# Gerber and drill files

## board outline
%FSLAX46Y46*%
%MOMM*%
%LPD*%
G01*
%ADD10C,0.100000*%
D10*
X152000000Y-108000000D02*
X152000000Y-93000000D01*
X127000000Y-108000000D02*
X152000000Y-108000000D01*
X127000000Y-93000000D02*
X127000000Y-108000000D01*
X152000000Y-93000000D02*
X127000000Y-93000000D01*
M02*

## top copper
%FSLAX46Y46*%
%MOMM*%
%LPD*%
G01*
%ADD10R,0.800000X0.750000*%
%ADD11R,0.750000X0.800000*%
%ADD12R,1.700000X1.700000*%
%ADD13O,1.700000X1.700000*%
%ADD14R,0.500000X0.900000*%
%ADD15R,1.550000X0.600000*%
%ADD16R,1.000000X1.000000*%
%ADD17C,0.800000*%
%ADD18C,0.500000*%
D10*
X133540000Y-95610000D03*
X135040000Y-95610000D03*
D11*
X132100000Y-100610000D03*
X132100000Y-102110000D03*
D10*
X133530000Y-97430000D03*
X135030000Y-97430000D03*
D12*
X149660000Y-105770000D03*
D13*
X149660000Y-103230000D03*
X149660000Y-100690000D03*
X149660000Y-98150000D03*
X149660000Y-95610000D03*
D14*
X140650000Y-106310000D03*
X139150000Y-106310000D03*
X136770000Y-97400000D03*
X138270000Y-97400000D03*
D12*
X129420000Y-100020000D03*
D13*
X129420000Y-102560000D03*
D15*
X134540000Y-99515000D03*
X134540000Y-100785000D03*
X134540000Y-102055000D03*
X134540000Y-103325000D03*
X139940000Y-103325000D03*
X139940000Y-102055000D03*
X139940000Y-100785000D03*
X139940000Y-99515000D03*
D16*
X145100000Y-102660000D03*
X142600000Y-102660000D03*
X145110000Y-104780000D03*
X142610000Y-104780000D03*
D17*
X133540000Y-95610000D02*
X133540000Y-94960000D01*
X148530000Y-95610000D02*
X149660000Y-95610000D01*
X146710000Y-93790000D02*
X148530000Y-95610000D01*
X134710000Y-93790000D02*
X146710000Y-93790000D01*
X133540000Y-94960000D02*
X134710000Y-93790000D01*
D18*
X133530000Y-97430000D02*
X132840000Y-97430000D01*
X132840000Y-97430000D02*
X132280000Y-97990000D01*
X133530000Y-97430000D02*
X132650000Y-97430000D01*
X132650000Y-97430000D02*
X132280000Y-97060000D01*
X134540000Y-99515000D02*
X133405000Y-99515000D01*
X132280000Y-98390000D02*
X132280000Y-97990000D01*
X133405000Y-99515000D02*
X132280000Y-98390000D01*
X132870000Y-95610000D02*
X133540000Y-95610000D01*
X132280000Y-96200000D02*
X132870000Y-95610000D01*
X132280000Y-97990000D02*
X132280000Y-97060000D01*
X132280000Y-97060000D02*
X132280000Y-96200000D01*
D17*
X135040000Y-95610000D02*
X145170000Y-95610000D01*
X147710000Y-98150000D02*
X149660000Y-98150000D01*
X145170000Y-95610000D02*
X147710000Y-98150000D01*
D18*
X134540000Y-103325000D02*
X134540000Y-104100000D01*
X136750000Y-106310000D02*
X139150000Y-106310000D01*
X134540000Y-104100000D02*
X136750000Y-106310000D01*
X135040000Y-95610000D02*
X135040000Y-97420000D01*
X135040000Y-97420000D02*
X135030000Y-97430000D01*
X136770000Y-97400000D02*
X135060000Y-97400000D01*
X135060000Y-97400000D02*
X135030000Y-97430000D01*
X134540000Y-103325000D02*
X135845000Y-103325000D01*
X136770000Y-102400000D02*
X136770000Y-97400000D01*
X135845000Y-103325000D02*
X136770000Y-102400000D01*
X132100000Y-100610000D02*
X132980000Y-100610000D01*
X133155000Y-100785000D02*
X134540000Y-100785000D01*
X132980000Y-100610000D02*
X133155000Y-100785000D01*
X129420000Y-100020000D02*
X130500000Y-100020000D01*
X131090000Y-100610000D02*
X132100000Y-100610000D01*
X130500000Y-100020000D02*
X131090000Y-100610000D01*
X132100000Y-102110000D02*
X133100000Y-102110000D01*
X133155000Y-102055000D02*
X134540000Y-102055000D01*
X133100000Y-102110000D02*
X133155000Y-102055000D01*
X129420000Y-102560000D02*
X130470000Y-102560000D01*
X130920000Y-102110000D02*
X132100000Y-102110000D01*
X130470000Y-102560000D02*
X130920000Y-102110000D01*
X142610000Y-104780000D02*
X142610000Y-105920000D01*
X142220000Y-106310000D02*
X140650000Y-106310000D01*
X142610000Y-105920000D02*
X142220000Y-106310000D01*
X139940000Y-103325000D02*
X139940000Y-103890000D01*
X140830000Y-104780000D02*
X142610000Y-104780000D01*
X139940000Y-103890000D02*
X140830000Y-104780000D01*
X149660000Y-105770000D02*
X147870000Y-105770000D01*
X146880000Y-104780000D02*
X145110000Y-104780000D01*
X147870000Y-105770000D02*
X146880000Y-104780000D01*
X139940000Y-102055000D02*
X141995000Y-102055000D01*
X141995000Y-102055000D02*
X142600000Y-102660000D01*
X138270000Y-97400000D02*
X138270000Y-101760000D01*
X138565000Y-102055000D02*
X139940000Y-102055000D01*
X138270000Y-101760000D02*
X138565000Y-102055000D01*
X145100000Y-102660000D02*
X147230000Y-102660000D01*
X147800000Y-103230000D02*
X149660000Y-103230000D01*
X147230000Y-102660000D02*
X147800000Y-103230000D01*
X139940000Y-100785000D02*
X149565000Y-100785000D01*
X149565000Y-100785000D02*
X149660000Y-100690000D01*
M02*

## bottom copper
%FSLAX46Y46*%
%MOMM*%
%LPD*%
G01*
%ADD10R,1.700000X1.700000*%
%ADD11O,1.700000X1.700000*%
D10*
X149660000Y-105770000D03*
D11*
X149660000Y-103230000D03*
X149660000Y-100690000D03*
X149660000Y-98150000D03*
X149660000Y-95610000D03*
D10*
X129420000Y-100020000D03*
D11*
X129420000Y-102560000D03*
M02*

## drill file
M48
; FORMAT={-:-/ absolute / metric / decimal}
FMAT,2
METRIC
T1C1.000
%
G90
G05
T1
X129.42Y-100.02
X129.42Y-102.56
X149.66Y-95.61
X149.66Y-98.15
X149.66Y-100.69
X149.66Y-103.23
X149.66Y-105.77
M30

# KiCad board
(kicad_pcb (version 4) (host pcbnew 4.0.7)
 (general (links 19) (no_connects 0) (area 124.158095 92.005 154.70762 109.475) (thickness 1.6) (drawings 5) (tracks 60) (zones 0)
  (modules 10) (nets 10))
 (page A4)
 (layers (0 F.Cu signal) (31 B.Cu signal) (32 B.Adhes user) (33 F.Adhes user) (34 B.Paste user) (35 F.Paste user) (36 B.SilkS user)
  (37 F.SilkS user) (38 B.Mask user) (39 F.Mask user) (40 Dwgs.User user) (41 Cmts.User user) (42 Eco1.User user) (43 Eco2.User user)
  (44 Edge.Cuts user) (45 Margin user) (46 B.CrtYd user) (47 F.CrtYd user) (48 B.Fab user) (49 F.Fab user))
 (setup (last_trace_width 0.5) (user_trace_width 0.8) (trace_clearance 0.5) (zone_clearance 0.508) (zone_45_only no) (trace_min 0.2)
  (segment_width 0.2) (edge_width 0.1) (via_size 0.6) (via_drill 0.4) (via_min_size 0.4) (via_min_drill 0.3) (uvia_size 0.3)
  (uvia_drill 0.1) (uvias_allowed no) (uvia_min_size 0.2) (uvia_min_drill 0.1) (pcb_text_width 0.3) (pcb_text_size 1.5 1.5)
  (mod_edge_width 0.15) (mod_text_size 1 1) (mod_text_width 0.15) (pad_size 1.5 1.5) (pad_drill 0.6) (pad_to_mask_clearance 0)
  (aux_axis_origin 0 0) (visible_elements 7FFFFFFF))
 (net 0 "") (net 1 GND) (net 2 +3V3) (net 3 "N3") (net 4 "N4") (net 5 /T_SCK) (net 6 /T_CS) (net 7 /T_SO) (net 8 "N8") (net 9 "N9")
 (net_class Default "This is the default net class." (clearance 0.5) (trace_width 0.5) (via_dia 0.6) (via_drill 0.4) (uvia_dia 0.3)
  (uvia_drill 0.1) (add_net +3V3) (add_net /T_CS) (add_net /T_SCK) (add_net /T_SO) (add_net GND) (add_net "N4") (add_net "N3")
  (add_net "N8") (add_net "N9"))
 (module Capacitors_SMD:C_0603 (layer F.Cu) (at 134.29 95.61 180)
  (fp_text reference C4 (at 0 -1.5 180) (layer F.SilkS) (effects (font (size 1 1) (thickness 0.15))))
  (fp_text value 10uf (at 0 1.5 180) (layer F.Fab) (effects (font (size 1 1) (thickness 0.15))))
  (pad 2 smd rect (at 0.75 0 180) (size 0.8 0.75) (layers F.Cu F.Paste F.Mask) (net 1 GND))
  (pad 1 smd rect (at -0.75 0 180) (size 0.8 0.75) (layers F.Cu F.Paste F.Mask) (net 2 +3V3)))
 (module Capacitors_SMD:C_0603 (layer F.Cu) (at 132.1 101.36 90)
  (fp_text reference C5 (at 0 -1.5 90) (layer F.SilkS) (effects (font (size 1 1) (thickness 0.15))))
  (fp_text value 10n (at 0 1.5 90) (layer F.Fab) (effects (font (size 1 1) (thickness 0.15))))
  (pad 2 smd rect (at 0.75 0 90) (size 0.8 0.75) (layers F.Cu F.Paste F.Mask) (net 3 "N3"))
  (pad 1 smd rect (at -0.75 0 90) (size 0.8 0.75) (layers F.Cu F.Paste F.Mask) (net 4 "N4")))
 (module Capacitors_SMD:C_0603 (layer F.Cu) (at 134.28 97.43 180)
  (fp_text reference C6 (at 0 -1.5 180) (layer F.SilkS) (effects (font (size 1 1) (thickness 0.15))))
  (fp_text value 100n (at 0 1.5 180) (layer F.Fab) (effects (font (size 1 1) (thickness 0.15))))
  (pad 2 smd rect (at 0.75 0 180) (size 0.8 0.75) (layers F.Cu F.Paste F.Mask) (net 1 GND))
  (pad 1 smd rect (at -0.75 0 180) (size 0.8 0.75) (layers F.Cu F.Paste F.Mask) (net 2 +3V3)))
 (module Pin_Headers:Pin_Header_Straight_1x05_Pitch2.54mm (layer F.Cu) (at 149.66 105.77 180)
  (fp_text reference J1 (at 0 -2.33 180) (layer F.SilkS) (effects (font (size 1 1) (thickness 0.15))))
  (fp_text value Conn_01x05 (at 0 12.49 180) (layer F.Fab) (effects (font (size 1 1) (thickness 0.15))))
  (pad 1 thru_hole rect (at 0 0 180) (size 1.7 1.7) (drill 1) (layers *.Cu *.Mask) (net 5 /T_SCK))
  (pad 2 thru_hole oval (at 0 2.54 180) (size 1.7 1.7) (drill 1) (layers *.Cu *.Mask) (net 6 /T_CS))
  (pad 3 thru_hole oval (at 0 5.08 180) (size 1.7 1.7) (drill 1) (layers *.Cu *.Mask) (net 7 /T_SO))
  (pad 4 thru_hole oval (at 0 7.62 180) (size 1.7 1.7) (drill 1) (layers *.Cu *.Mask) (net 2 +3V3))
  (pad 5 thru_hole oval (at 0 10.16 180) (size 1.7 1.7) (drill 1) (layers *.Cu *.Mask) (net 1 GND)))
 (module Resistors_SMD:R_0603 (layer F.Cu) (at 139.9 106.31 180)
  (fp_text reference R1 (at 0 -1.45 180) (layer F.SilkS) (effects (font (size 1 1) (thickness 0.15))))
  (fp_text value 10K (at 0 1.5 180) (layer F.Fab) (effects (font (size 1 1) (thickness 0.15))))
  (pad 1 smd rect (at -0.75 0 180) (size 0.5 0.9) (layers F.Cu F.Paste F.Mask) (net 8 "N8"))
  (pad 2 smd rect (at 0.75 0 180) (size 0.5 0.9) (layers F.Cu F.Paste F.Mask) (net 2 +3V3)))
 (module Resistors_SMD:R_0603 (layer F.Cu) (at 137.52 97.4)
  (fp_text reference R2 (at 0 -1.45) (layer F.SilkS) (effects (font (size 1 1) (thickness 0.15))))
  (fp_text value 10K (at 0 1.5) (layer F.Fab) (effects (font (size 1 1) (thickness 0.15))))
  (pad 1 smd rect (at -0.75 0) (size 0.5 0.9) (layers F.Cu F.Paste F.Mask) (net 2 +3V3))
  (pad 2 smd rect (at 0.75 0) (size 0.5 0.9) (layers F.Cu F.Paste F.Mask) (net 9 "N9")))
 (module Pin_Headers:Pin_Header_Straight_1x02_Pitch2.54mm (layer F.Cu) (at 129.42 100.02)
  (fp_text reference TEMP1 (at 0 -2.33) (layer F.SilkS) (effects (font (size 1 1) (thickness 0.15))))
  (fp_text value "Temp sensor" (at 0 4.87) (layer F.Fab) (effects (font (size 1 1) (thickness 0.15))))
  (pad 1 thru_hole rect (at 0 0) (size 1.7 1.7) (drill 1) (layers *.Cu *.Mask) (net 3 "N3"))
  (pad 2 thru_hole oval (at 0 2.54) (size 1.7 1.7) (drill 1) (layers *.Cu *.Mask) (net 4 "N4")))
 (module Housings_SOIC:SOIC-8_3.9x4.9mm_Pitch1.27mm (layer F.Cu) (at 137.24 101.42)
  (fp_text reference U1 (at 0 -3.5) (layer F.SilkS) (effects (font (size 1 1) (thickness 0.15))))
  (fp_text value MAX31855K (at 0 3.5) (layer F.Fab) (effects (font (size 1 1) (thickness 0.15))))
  (pad 1 smd rect (at -2.7 -1.905) (size 1.55 0.6) (layers F.Cu F.Paste F.Mask) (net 1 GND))
  (pad 2 smd rect (at -2.7 -0.635) (size 1.55 0.6) (layers F.Cu F.Paste F.Mask) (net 3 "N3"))
  (pad 3 smd rect (at -2.7 0.635) (size 1.55 0.6) (layers F.Cu F.Paste F.Mask) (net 4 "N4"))
  (pad 4 smd rect (at -2.7 1.905) (size 1.55 0.6) (layers F.Cu F.Paste F.Mask) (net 2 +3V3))
  (pad 5 smd rect (at 2.7 1.905) (size 1.55 0.6) (layers F.Cu F.Paste F.Mask) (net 8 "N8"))
  (pad 6 smd rect (at 2.7 0.635) (size 1.55 0.6) (layers F.Cu F.Paste F.Mask) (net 9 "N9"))
  (pad 7 smd rect (at 2.7 -0.635) (size 1.55 0.6) (layers F.Cu F.Paste F.Mask) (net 7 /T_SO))
  (pad 8 smd rect (at 2.7 -1.905) (size 1.55 0.6) (layers F.Cu F.Paste F.Mask)))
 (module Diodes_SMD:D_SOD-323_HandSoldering (layer F.Cu) (at 143.85 102.66 180)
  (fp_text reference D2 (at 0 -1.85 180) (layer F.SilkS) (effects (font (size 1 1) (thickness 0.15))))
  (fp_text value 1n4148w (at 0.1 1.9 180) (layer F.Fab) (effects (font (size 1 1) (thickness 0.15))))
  (pad 1 smd rect (at -1.25 0 180) (size 1 1) (layers F.Cu F.Paste F.Mask) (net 6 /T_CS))
  (pad 2 smd rect (at 1.25 0 180) (size 1 1) (layers F.Cu F.Paste F.Mask) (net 9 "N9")))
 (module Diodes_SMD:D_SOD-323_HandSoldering (layer F.Cu) (at 143.86 104.78 180)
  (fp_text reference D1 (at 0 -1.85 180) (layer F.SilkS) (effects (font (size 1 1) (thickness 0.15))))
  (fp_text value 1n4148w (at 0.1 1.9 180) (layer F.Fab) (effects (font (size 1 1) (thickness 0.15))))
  (pad 1 smd rect (at -1.25 0 180) (size 1 1) (layers F.Cu F.Paste F.Mask) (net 5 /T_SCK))
  (pad 2 smd rect (at 1.25 0 180) (size 1 1) (layers F.Cu F.Paste F.Mask) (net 8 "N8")))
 (gr_line (start 152 108) (end 152 93) (angle 90) (layer Edge.Cuts) (width 0.1))
 (gr_line (start 127 108) (end 152 108) (angle 90) (layer Edge.Cuts) (width 0.1))
 (gr_line (start 127 93) (end 127 108) (angle 90) (layer Edge.Cuts) (width 0.1))
 (gr_line (start 152 93) (end 127 93) (angle 90) (layer Edge.Cuts) (width 0.1))
 (segment (start 133.54 95.61) (end 133.54 94.96) (width 0.8) (layer F.Cu) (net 1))
 (segment (start 148.53 95.61) (end 149.66 95.61) (width 0.8) (layer F.Cu) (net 1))
 (segment (start 146.71 93.79) (end 148.53 95.61) (width 0.8) (layer F.Cu) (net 1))
 (segment (start 134.71 93.79) (end 146.71 93.79) (width 0.8) (layer F.Cu) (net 1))
 (segment (start 133.54 94.96) (end 134.71 93.79) (width 0.8) (layer F.Cu) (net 1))
 (segment (start 133.53 97.43) (end 132.84 97.43) (width 0.5) (layer F.Cu) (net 1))
 (segment (start 132.84 97.43) (end 132.28 97.99) (width 0.5) (layer F.Cu) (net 1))
 (segment (start 133.53 97.43) (end 132.65 97.43) (width 0.5) (layer F.Cu) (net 1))
 (segment (start 132.65 97.43) (end 132.28 97.06) (width 0.5) (layer F.Cu) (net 1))
 (segment (start 134.54 99.515) (end 133.405 99.515) (width 0.5) (layer F.Cu) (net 1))
 (segment (start 132.28 98.39) (end 132.28 97.99) (width 0.5) (layer F.Cu) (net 1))
 (segment (start 133.405 99.515) (end 132.28 98.39) (width 0.5) (layer F.Cu) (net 1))
 (segment (start 132.87 95.61) (end 133.54 95.61) (width 0.5) (layer F.Cu) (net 1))
 (segment (start 132.28 96.2) (end 132.87 95.61) (width 0.5) (layer F.Cu) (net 1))
 (segment (start 132.28 97.99) (end 132.28 97.06) (width 0.5) (layer F.Cu) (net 1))
 (segment (start 132.28 97.06) (end 132.28 96.2) (width 0.5) (layer F.Cu) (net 1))
 (segment (start 135.04 95.61) (end 145.17 95.61) (width 0.8) (layer F.Cu) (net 2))
 (segment (start 147.71 98.15) (end 149.66 98.15) (width 0.8) (layer F.Cu) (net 2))
 (segment (start 145.17 95.61) (end 147.71 98.15) (width 0.8) (layer F.Cu) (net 2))
 (segment (start 134.54 103.325) (end 134.54 104.1) (width 0.5) (layer F.Cu) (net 2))
 (segment (start 136.75 106.31) (end 139.15 106.31) (width 0.5) (layer F.Cu) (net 2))
 (segment (start 134.54 104.1) (end 136.75 106.31) (width 0.5) (layer F.Cu) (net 2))
 (segment (start 135.04 95.61) (end 135.04 97.42) (width 0.5) (layer F.Cu) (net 2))
 (segment (start 135.04 97.42) (end 135.03 97.43) (width 0.5) (layer F.Cu) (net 2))
 (segment (start 136.77 97.4) (end 135.06 97.4) (width 0.5) (layer F.Cu) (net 2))
 (segment (start 135.06 97.4) (end 135.03 97.43) (width 0.5) (layer F.Cu) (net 2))
 (segment (start 134.54 103.325) (end 135.845 103.325) (width 0.5) (layer F.Cu) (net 2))
 (segment (start 136.77 102.4) (end 136.77 97.4) (width 0.5) (layer F.Cu) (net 2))
 (segment (start 135.845 103.325) (end 136.77 102.4) (width 0.5) (layer F.Cu) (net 2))
 (segment (start 132.1 100.61) (end 132.98 100.61) (width 0.5) (layer F.Cu) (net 3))
 (segment (start 133.155 100.785) (end 134.54 100.785) (width 0.5) (layer F.Cu) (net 3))
 (segment (start 132.98 100.61) (end 133.155 100.785) (width 0.5) (layer F.Cu) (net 3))
 (segment (start 129.42 100.02) (end 130.5 100.02) (width 0.5) (layer F.Cu) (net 3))
 (segment (start 131.09 100.61) (end 132.1 100.61) (width 0.5) (layer F.Cu) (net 3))
 (segment (start 130.5 100.02) (end 131.09 100.61) (width 0.5) (layer F.Cu) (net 3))
 (segment (start 132.1 102.11) (end 133.1 102.11) (width 0.5) (layer F.Cu) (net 4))
 (segment (start 133.155 102.055) (end 134.54 102.055) (width 0.5) (layer F.Cu) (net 4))
 (segment (start 133.1 102.11) (end 133.155 102.055) (width 0.5) (layer F.Cu) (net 4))
 (segment (start 129.42 102.56) (end 130.47 102.56) (width 0.5) (layer F.Cu) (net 4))
 (segment (start 130.92 102.11) (end 132.1 102.11) (width 0.5) (layer F.Cu) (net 4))
 (segment (start 130.47 102.56) (end 130.92 102.11) (width 0.5) (layer F.Cu) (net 4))
 (segment (start 142.61 104.78) (end 142.61 105.92) (width 0.5) (layer F.Cu) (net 8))
 (segment (start 142.22 106.31) (end 140.65 106.31) (width 0.5) (layer F.Cu) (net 8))
 (segment (start 142.61 105.92) (end 142.22 106.31) (width 0.5) (layer F.Cu) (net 8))
 (segment (start 139.94 103.325) (end 139.94 103.89) (width 0.5) (layer F.Cu) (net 8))
 (segment (start 140.83 104.78) (end 142.61 104.78) (width 0.5) (layer F.Cu) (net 8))
 (segment (start 139.94 103.89) (end 140.83 104.78) (width 0.5) (layer F.Cu) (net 8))
 (segment (start 149.66 105.77) (end 147.87 105.77) (width 0.5) (layer F.Cu) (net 5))
 (segment (start 146.88 104.78) (end 145.11 104.78) (width 0.5) (layer F.Cu) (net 5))
 (segment (start 147.87 105.77) (end 146.88 104.78) (width 0.5) (layer F.Cu) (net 5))
 (segment (start 139.94 102.055) (end 141.995 102.055) (width 0.5) (layer F.Cu) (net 9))
 (segment (start 141.995 102.055) (end 142.6 102.66) (width 0.5) (layer F.Cu) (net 9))
 (segment (start 138.27 97.4) (end 138.27 101.76) (width 0.5) (layer F.Cu) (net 9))
 (segment (start 138.565 102.055) (end 139.94 102.055) (width 0.5) (layer F.Cu) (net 9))
 (segment (start 138.27 101.76) (end 138.565 102.055) (width 0.5) (layer F.Cu) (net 9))
 (segment (start 145.1 102.66) (end 147.23 102.66) (width 0.5) (layer F.Cu) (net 6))
 (segment (start 147.8 103.23) (end 149.66 103.23) (width 0.5) (layer F.Cu) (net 6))
 (segment (start 147.23 102.66) (end 147.8 103.23) (width 0.5) (layer F.Cu) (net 6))
 (segment (start 139.94 100.785) (end 149.565 100.785) (width 0.5) (layer F.Cu) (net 7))
 (segment (start 149.565 100.785) (end 149.66 100.69) (width 0.5) (layer F.Cu) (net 7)))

